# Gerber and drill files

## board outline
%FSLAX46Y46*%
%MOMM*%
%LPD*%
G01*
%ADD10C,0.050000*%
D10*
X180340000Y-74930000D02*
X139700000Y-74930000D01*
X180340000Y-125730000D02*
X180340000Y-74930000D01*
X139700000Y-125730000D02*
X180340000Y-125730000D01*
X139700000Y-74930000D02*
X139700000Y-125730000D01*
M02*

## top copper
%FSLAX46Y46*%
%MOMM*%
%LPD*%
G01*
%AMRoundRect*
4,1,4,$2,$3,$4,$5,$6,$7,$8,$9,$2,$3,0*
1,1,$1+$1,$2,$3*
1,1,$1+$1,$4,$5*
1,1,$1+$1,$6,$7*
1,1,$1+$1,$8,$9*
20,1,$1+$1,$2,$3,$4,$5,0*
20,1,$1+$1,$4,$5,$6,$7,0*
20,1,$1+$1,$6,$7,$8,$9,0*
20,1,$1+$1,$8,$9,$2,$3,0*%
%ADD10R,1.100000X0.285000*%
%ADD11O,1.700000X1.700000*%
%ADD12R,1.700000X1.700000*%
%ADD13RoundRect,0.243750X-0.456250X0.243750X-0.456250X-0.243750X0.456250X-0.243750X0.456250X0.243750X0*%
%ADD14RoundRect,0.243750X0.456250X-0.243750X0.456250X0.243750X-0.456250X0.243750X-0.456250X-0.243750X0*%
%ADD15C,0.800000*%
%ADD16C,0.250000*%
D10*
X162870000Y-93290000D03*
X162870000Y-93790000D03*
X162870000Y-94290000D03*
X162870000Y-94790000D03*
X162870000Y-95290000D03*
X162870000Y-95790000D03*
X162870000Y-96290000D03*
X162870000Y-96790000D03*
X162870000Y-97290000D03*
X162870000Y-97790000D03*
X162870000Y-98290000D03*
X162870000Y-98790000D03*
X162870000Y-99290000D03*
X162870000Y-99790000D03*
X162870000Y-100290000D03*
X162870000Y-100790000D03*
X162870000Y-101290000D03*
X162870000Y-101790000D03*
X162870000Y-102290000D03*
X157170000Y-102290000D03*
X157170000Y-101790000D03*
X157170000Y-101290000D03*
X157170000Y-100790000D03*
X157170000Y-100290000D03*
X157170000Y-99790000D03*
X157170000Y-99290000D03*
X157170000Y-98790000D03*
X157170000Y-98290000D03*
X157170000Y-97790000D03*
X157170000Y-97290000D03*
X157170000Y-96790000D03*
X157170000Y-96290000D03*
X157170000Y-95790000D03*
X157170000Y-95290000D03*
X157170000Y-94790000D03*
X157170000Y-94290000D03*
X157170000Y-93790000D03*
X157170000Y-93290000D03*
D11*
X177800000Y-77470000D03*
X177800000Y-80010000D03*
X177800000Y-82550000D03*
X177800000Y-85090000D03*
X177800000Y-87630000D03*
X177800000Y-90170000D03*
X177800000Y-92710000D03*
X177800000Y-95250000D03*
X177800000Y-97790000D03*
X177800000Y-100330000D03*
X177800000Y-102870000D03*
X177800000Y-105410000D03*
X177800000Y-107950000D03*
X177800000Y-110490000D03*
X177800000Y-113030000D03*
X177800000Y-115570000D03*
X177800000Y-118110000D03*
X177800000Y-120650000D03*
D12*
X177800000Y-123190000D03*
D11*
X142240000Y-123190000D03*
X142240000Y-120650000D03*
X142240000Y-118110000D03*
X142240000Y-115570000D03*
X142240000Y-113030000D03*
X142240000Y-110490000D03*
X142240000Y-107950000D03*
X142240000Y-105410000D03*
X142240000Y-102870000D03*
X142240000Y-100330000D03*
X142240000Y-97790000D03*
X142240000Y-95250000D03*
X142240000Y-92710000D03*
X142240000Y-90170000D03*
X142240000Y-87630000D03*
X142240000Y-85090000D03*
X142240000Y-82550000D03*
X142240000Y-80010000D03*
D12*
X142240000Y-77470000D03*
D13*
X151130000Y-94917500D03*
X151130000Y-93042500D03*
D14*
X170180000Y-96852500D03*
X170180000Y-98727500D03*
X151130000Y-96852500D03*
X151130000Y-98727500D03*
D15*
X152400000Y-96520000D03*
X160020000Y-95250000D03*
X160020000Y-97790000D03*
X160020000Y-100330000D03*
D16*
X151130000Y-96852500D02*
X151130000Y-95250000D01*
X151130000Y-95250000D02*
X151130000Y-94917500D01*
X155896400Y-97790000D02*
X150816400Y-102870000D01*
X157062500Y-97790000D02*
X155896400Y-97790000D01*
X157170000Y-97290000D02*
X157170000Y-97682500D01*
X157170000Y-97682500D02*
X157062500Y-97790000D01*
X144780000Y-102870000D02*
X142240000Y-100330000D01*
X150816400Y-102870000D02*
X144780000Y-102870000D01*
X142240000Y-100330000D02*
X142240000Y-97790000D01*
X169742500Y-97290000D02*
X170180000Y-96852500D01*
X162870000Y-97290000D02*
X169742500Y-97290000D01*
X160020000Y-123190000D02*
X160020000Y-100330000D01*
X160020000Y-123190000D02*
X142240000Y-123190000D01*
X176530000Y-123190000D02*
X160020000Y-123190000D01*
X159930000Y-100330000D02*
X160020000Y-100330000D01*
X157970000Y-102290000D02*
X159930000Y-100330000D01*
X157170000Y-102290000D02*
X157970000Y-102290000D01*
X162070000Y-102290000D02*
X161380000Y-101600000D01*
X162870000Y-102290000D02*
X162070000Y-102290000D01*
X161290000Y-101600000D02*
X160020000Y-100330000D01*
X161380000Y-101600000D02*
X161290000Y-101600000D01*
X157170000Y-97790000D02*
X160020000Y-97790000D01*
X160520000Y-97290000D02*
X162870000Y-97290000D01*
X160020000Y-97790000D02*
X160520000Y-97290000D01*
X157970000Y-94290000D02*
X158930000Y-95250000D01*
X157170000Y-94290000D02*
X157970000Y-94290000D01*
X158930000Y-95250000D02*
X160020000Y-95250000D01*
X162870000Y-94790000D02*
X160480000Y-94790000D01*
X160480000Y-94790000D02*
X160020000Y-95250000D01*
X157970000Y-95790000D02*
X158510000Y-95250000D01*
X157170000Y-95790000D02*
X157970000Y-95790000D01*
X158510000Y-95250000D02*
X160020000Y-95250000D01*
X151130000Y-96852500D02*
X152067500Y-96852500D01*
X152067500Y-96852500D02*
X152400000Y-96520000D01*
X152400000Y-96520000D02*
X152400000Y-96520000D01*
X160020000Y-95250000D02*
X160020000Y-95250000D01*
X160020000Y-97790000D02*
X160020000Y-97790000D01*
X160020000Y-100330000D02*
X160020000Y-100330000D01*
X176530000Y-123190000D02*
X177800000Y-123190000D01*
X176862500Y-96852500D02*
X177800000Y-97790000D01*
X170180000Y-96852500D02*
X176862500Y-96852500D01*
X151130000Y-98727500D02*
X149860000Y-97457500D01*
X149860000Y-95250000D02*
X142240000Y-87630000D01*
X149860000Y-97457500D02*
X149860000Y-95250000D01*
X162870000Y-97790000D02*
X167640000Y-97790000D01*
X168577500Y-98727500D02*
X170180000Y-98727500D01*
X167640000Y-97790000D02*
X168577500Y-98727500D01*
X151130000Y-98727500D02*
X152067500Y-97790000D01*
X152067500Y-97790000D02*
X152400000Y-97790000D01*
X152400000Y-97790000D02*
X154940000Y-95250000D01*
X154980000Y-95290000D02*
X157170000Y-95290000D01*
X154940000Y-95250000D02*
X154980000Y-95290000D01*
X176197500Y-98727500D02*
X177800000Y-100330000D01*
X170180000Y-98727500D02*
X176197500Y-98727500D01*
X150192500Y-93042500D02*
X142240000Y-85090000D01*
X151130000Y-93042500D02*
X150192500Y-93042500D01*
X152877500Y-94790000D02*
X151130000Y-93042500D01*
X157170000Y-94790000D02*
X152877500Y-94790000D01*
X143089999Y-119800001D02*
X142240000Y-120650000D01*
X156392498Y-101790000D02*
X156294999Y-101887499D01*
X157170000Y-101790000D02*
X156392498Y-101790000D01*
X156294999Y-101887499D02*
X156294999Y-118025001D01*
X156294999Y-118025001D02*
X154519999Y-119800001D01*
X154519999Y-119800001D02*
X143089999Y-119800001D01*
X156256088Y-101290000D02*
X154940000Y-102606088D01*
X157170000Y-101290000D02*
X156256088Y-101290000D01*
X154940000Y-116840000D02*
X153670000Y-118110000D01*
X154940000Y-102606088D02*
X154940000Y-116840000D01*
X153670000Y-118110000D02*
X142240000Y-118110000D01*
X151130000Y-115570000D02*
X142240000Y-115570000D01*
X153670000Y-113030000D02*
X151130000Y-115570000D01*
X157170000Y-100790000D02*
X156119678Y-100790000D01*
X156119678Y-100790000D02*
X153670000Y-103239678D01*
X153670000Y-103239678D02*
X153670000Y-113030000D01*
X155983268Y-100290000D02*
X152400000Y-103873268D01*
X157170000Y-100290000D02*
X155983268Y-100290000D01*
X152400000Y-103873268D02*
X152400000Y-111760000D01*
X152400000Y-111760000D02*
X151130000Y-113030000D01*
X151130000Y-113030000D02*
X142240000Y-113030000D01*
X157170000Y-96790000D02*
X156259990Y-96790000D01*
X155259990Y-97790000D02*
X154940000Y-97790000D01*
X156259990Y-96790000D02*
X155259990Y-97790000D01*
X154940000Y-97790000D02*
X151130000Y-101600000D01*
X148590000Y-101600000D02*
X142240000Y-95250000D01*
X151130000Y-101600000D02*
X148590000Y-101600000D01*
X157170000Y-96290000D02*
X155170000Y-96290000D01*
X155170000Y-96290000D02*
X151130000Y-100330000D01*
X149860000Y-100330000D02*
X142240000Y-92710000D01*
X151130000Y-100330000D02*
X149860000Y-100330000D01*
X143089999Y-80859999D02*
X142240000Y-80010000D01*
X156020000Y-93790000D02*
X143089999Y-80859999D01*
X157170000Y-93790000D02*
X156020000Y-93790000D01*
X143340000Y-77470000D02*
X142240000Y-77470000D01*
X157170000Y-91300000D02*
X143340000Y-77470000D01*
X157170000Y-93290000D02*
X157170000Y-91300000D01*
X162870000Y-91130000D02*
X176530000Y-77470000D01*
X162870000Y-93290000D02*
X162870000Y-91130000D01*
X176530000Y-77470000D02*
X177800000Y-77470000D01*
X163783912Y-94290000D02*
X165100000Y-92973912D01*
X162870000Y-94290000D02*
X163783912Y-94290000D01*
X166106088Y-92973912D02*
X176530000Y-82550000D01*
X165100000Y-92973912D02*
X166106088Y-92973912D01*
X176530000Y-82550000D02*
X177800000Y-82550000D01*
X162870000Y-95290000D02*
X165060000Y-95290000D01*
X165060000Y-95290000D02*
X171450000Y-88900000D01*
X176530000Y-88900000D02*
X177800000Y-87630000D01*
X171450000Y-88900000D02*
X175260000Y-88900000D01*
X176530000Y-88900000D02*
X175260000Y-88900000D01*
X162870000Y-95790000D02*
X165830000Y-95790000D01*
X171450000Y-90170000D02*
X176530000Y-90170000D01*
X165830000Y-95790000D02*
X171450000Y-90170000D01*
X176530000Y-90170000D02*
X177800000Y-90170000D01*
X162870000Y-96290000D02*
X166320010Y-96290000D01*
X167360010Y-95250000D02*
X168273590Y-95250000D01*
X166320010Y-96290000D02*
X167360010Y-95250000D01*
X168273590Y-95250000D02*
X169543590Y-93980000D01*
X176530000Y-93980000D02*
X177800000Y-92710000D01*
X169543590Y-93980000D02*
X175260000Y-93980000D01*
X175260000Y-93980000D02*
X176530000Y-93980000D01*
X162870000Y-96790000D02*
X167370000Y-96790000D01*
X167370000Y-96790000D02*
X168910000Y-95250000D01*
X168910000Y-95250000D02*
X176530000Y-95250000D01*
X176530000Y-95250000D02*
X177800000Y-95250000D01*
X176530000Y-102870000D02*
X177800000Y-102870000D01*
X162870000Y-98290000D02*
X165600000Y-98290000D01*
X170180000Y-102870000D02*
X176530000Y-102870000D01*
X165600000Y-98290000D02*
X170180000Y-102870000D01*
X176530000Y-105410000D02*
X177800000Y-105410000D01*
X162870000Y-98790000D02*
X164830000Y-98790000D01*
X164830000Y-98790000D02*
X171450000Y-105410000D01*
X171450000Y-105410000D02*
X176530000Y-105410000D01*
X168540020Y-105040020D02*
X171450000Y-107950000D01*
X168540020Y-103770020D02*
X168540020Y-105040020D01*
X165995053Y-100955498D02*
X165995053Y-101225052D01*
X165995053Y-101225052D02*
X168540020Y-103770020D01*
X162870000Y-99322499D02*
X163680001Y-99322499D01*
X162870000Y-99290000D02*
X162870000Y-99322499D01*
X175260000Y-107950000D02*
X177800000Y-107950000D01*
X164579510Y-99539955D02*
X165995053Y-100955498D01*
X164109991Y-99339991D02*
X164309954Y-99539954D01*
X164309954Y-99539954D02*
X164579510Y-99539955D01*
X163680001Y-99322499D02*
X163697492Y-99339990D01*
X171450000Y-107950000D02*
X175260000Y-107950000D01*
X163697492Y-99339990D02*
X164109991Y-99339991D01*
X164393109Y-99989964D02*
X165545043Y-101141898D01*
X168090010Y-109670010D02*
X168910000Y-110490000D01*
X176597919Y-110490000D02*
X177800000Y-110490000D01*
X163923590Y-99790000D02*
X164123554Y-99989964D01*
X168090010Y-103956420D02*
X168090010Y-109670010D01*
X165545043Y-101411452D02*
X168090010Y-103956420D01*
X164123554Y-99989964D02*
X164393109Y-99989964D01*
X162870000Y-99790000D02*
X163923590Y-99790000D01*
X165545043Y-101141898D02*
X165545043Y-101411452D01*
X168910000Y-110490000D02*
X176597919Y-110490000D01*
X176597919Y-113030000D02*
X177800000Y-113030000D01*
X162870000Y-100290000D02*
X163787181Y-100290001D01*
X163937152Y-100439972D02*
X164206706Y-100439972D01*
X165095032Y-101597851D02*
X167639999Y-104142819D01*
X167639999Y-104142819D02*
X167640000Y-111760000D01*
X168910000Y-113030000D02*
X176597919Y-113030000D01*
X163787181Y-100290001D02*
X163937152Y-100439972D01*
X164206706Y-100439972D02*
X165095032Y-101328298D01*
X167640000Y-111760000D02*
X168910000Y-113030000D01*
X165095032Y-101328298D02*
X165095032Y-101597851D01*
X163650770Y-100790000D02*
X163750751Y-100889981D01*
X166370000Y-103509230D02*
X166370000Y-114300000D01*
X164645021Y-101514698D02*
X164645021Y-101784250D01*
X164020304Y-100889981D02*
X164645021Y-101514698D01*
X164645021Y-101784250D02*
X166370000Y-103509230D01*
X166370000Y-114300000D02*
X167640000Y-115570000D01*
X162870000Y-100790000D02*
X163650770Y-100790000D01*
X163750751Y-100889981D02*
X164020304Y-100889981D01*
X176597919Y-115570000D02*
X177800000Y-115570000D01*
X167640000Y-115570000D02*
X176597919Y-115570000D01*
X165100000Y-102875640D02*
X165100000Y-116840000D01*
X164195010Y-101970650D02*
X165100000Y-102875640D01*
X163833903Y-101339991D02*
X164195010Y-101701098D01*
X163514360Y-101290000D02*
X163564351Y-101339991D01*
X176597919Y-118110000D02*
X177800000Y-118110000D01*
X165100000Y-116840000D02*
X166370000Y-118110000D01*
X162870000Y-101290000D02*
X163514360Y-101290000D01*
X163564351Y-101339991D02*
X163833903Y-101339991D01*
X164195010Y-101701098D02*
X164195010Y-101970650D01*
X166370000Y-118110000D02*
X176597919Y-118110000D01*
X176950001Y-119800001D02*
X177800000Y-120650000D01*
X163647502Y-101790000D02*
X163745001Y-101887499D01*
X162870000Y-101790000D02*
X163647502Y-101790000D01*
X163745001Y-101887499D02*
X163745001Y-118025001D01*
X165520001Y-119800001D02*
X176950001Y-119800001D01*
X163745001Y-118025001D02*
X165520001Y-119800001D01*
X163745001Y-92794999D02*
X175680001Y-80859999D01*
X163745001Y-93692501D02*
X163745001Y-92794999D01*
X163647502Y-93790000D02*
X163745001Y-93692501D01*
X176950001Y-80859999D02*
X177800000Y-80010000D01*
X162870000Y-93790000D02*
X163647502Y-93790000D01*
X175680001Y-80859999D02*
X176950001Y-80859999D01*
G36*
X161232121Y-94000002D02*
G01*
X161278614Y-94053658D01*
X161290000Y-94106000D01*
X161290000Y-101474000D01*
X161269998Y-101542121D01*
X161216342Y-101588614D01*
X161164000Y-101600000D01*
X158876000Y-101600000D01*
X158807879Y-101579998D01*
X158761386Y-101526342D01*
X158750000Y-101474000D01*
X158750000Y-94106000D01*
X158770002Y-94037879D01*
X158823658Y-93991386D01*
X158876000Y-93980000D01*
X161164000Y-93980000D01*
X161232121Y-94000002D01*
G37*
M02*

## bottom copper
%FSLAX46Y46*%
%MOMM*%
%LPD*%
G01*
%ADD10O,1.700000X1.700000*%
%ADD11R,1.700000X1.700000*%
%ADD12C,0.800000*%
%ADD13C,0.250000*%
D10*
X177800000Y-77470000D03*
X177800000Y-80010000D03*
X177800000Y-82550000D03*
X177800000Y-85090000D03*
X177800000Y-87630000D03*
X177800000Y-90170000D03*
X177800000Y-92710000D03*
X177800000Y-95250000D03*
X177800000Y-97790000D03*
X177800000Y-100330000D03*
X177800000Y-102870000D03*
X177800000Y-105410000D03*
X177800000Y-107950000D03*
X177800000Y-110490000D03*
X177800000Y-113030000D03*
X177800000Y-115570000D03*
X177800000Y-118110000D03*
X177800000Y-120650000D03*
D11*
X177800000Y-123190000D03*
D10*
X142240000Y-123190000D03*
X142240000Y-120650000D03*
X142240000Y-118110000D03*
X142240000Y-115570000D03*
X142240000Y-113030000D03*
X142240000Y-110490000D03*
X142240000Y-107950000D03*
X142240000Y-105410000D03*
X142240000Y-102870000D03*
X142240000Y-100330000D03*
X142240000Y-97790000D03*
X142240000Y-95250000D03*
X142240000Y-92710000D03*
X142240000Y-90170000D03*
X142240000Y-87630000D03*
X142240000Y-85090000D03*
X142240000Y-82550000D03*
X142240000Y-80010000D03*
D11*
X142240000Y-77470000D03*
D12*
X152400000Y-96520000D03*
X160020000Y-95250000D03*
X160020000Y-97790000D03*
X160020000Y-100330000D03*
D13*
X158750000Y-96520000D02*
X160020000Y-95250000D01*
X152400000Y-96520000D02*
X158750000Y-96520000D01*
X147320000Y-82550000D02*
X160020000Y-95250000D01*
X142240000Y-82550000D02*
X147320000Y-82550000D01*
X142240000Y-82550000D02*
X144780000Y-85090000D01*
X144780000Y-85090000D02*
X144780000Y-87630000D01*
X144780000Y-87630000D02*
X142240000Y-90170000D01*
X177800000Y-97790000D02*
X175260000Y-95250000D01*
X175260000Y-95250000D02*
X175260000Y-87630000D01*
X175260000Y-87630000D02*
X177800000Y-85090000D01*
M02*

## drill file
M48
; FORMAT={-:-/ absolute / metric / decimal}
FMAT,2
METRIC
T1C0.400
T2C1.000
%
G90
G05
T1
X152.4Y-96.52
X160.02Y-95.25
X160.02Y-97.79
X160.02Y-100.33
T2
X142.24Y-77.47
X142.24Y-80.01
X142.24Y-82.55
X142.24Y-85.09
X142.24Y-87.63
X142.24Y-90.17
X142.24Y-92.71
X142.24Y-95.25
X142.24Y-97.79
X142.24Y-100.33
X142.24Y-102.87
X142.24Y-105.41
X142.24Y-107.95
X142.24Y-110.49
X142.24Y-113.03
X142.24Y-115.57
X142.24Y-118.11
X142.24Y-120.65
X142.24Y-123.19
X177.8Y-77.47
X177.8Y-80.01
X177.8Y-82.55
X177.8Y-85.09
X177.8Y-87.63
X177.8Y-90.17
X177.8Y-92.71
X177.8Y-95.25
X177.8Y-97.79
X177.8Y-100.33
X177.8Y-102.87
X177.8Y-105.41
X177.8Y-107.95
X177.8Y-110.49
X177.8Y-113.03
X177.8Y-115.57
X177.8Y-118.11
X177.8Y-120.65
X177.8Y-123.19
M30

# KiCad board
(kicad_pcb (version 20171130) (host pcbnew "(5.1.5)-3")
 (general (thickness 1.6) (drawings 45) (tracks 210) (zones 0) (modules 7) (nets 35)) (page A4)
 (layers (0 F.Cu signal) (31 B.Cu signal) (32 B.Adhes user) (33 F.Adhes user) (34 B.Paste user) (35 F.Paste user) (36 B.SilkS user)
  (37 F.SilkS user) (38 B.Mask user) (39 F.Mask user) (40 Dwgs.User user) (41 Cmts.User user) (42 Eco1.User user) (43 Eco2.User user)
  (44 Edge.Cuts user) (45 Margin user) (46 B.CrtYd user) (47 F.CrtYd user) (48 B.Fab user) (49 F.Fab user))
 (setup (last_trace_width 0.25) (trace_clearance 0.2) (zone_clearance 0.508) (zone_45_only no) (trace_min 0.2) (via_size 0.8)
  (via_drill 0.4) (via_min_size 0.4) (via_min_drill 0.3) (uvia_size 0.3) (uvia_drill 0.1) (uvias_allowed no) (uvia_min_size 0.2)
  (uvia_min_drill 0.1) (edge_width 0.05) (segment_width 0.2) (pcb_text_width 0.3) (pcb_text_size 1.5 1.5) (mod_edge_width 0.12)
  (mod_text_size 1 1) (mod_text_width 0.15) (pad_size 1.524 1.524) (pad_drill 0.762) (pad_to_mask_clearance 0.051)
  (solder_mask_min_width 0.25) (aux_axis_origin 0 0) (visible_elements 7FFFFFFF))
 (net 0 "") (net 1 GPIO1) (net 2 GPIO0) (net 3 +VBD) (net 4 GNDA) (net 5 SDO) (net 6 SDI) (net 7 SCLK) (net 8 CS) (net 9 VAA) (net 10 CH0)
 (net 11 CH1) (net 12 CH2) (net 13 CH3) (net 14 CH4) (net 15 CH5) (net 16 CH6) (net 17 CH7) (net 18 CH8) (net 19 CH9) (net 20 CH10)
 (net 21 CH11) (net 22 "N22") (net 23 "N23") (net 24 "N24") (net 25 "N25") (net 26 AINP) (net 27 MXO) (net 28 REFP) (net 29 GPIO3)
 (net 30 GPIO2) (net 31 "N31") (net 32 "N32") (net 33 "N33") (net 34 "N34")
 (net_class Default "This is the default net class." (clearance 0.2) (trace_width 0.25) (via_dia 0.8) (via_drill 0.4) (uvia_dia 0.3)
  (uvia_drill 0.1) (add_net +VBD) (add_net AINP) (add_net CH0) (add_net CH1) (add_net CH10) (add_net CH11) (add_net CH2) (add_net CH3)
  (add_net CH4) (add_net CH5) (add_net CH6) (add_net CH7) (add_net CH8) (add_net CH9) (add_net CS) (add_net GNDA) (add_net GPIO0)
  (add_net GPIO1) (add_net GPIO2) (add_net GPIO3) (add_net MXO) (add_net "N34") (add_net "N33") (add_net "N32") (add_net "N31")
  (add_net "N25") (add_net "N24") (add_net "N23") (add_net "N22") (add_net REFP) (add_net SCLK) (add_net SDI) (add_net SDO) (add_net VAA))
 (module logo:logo (layer F.Cu) (at 160.02 82.55)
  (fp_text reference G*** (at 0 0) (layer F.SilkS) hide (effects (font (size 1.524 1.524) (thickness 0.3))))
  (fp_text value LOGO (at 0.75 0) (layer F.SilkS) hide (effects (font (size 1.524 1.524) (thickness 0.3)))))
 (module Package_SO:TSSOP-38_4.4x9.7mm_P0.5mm (layer F.Cu) (at 160.02 97.79)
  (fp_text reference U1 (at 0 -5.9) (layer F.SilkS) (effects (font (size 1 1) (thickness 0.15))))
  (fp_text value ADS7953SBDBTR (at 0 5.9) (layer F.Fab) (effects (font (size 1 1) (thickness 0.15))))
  (pad 38 smd rect (at 2.85 -4.5) (size 1.1 0.285) (layers F.Cu F.Paste F.Mask) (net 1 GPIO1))
  (pad 37 smd rect (at 2.85 -4) (size 1.1 0.285) (layers F.Cu F.Paste F.Mask) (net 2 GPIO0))
  (pad 36 smd rect (at 2.85 -3.5) (size 1.1 0.285) (layers F.Cu F.Paste F.Mask) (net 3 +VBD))
  (pad 35 smd rect (at 2.85 -3) (size 1.1 0.285) (layers F.Cu F.Paste F.Mask) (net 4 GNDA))
  (pad 34 smd rect (at 2.85 -2.5) (size 1.1 0.285) (layers F.Cu F.Paste F.Mask) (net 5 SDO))
  (pad 33 smd rect (at 2.85 -2) (size 1.1 0.285) (layers F.Cu F.Paste F.Mask) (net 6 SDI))
  (pad 32 smd rect (at 2.85 -1.5) (size 1.1 0.285) (layers F.Cu F.Paste F.Mask) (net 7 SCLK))
  (pad 31 smd rect (at 2.85 -1) (size 1.1 0.285) (layers F.Cu F.Paste F.Mask) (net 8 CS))
  (pad 30 smd rect (at 2.85 -0.5) (size 1.1 0.285) (layers F.Cu F.Paste F.Mask) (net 4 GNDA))
  (pad 29 smd rect (at 2.85 0) (size 1.1 0.285) (layers F.Cu F.Paste F.Mask) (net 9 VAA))
  (pad 28 smd rect (at 2.85 0.5) (size 1.1 0.285) (layers F.Cu F.Paste F.Mask) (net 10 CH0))
  (pad 27 smd rect (at 2.85 1) (size 1.1 0.285) (layers F.Cu F.Paste F.Mask) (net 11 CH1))
  (pad 26 smd rect (at 2.85 1.5) (size 1.1 0.285) (layers F.Cu F.Paste F.Mask) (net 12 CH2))
  (pad 25 smd rect (at 2.85 2) (size 1.1 0.285) (layers F.Cu F.Paste F.Mask) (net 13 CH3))
  (pad 24 smd rect (at 2.85 2.5) (size 1.1 0.285) (layers F.Cu F.Paste F.Mask) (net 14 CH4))
  (pad 23 smd rect (at 2.85 3) (size 1.1 0.285) (layers F.Cu F.Paste F.Mask) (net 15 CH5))
  (pad 22 smd rect (at 2.85 3.5) (size 1.1 0.285) (layers F.Cu F.Paste F.Mask) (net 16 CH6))
  (pad 21 smd rect (at 2.85 4) (size 1.1 0.285) (layers F.Cu F.Paste F.Mask) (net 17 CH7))
  (pad 20 smd rect (at 2.85 4.5) (size 1.1 0.285) (layers F.Cu F.Paste F.Mask) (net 4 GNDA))
  (pad 19 smd rect (at -2.85 4.5) (size 1.1 0.285) (layers F.Cu F.Paste F.Mask) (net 4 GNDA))
  (pad 18 smd rect (at -2.85 4) (size 1.1 0.285) (layers F.Cu F.Paste F.Mask) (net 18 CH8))
  (pad 17 smd rect (at -2.85 3.5) (size 1.1 0.285) (layers F.Cu F.Paste F.Mask) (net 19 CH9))
  (pad 16 smd rect (at -2.85 3) (size 1.1 0.285) (layers F.Cu F.Paste F.Mask) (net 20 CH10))
  (pad 15 smd rect (at -2.85 2.5) (size 1.1 0.285) (layers F.Cu F.Paste F.Mask) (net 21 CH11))
  (pad 14 smd rect (at -2.85 2) (size 1.1 0.285) (layers F.Cu F.Paste F.Mask) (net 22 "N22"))
  (pad 13 smd rect (at -2.85 1.5) (size 1.1 0.285) (layers F.Cu F.Paste F.Mask) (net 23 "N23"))
  (pad 12 smd rect (at -2.85 1) (size 1.1 0.285) (layers F.Cu F.Paste F.Mask) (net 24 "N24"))
  (pad 11 smd rect (at -2.85 0.5) (size 1.1 0.285) (layers F.Cu F.Paste F.Mask) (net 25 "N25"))
  (pad 10 smd rect (at -2.85 0) (size 1.1 0.285) (layers F.Cu F.Paste F.Mask) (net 4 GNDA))
  (pad 9 smd rect (at -2.85 -0.5) (size 1.1 0.285) (layers F.Cu F.Paste F.Mask) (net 4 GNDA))
  (pad 8 smd rect (at -2.85 -1) (size 1.1 0.285) (layers F.Cu F.Paste F.Mask) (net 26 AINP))
  (pad 7 smd rect (at -2.85 -1.5) (size 1.1 0.285) (layers F.Cu F.Paste F.Mask) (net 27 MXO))
  (pad 6 smd rect (at -2.85 -2) (size 1.1 0.285) (layers F.Cu F.Paste F.Mask) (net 4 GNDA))
  (pad 5 smd rect (at -2.85 -2.5) (size 1.1 0.285) (layers F.Cu F.Paste F.Mask) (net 9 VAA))
  (pad 4 smd rect (at -2.85 -3) (size 1.1 0.285) (layers F.Cu F.Paste F.Mask) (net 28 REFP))
  (pad 3 smd rect (at -2.85 -3.5) (size 1.1 0.285) (layers F.Cu F.Paste F.Mask) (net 4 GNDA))
  (pad 2 smd rect (at -2.85 -4) (size 1.1 0.285) (layers F.Cu F.Paste F.Mask) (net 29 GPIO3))
  (pad 1 smd rect (at -2.85 -4.5) (size 1.1 0.285) (layers F.Cu F.Paste F.Mask) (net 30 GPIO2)))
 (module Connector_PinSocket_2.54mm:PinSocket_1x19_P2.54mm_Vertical (layer F.Cu) (at 177.8 123.19 180)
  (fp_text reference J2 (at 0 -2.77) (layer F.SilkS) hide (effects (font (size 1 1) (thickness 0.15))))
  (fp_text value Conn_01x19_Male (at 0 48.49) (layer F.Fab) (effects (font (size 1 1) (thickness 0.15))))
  (pad 19 thru_hole oval (at 0 45.72 180) (size 1.7 1.7) (drill 1) (layers *.Cu *.Mask) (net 1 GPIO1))
  (pad 18 thru_hole oval (at 0 43.18 180) (size 1.7 1.7) (drill 1) (layers *.Cu *.Mask) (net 2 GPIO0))
  (pad 17 thru_hole oval (at 0 40.64 180) (size 1.7 1.7) (drill 1) (layers *.Cu *.Mask) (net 3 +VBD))
  (pad 16 thru_hole oval (at 0 38.1 180) (size 1.7 1.7) (drill 1) (layers *.Cu *.Mask) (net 4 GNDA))
  (pad 15 thru_hole oval (at 0 35.56 180) (size 1.7 1.7) (drill 1) (layers *.Cu *.Mask) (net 5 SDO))
  (pad 14 thru_hole oval (at 0 33.02 180) (size 1.7 1.7) (drill 1) (layers *.Cu *.Mask) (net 6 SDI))
  (pad 13 thru_hole oval (at 0 30.48 180) (size 1.7 1.7) (drill 1) (layers *.Cu *.Mask) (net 7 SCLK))
  (pad 12 thru_hole oval (at 0 27.94 180) (size 1.7 1.7) (drill 1) (layers *.Cu *.Mask) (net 8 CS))
  (pad 11 thru_hole oval (at 0 25.4 180) (size 1.7 1.7) (drill 1) (layers *.Cu *.Mask) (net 4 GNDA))
  (pad 10 thru_hole oval (at 0 22.86 180) (size 1.7 1.7) (drill 1) (layers *.Cu *.Mask) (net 9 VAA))
  (pad 9 thru_hole oval (at 0 20.32 180) (size 1.7 1.7) (drill 1) (layers *.Cu *.Mask) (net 10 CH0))
  (pad 8 thru_hole oval (at 0 17.78 180) (size 1.7 1.7) (drill 1) (layers *.Cu *.Mask) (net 11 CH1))
  (pad 7 thru_hole oval (at 0 15.24 180) (size 1.7 1.7) (drill 1) (layers *.Cu *.Mask) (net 12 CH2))
  (pad 6 thru_hole oval (at 0 12.7 180) (size 1.7 1.7) (drill 1) (layers *.Cu *.Mask) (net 13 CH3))
  (pad 5 thru_hole oval (at 0 10.16 180) (size 1.7 1.7) (drill 1) (layers *.Cu *.Mask) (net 14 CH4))
  (pad 4 thru_hole oval (at 0 7.62 180) (size 1.7 1.7) (drill 1) (layers *.Cu *.Mask) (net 15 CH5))
  (pad 3 thru_hole oval (at 0 5.08 180) (size 1.7 1.7) (drill 1) (layers *.Cu *.Mask) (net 16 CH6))
  (pad 2 thru_hole oval (at 0 2.54 180) (size 1.7 1.7) (drill 1) (layers *.Cu *.Mask) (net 17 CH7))
  (pad 1 thru_hole rect (at 0 0 180) (size 1.7 1.7) (drill 1) (layers *.Cu *.Mask) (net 4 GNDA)))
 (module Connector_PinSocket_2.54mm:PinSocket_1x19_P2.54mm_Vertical (layer F.Cu) (at 142.24 77.47)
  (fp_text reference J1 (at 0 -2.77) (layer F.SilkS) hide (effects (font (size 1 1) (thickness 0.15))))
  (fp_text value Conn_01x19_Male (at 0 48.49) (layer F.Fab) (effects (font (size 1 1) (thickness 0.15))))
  (pad 19 thru_hole oval (at 0 45.72) (size 1.7 1.7) (drill 1) (layers *.Cu *.Mask) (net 4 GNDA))
  (pad 18 thru_hole oval (at 0 43.18) (size 1.7 1.7) (drill 1) (layers *.Cu *.Mask) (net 18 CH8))
  (pad 17 thru_hole oval (at 0 40.64) (size 1.7 1.7) (drill 1) (layers *.Cu *.Mask) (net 19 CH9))
  (pad 16 thru_hole oval (at 0 38.1) (size 1.7 1.7) (drill 1) (layers *.Cu *.Mask) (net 20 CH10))
  (pad 15 thru_hole oval (at 0 35.56) (size 1.7 1.7) (drill 1) (layers *.Cu *.Mask) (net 21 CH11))
  (pad 14 thru_hole oval (at 0 33.02) (size 1.7 1.7) (drill 1) (layers *.Cu *.Mask) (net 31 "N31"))
  (pad 13 thru_hole oval (at 0 30.48) (size 1.7 1.7) (drill 1) (layers *.Cu *.Mask) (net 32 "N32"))
  (pad 12 thru_hole oval (at 0 27.94) (size 1.7 1.7) (drill 1) (layers *.Cu *.Mask) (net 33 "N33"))
  (pad 11 thru_hole oval (at 0 25.4) (size 1.7 1.7) (drill 1) (layers *.Cu *.Mask) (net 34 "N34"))
  (pad 10 thru_hole oval (at 0 22.86) (size 1.7 1.7) (drill 1) (layers *.Cu *.Mask) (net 4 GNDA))
  (pad 9 thru_hole oval (at 0 20.32) (size 1.7 1.7) (drill 1) (layers *.Cu *.Mask) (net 4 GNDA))
  (pad 8 thru_hole oval (at 0 17.78) (size 1.7 1.7) (drill 1) (layers *.Cu *.Mask) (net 26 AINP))
  (pad 7 thru_hole oval (at 0 15.24) (size 1.7 1.7) (drill 1) (layers *.Cu *.Mask) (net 27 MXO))
  (pad 6 thru_hole oval (at 0 12.7) (size 1.7 1.7) (drill 1) (layers *.Cu *.Mask) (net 4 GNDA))
  (pad 5 thru_hole oval (at 0 10.16) (size 1.7 1.7) (drill 1) (layers *.Cu *.Mask) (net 9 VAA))
  (pad 4 thru_hole oval (at 0 7.62) (size 1.7 1.7) (drill 1) (layers *.Cu *.Mask) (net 28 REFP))
  (pad 3 thru_hole oval (at 0 5.08) (size 1.7 1.7) (drill 1) (layers *.Cu *.Mask) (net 4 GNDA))
  (pad 2 thru_hole oval (at 0 2.54) (size 1.7 1.7) (drill 1) (layers *.Cu *.Mask) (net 29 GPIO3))
  (pad 1 thru_hole rect (at 0 0) (size 1.7 1.7) (drill 1) (layers *.Cu *.Mask) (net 30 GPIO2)))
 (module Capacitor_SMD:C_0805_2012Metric (layer F.Cu) (at 151.13 93.98 270)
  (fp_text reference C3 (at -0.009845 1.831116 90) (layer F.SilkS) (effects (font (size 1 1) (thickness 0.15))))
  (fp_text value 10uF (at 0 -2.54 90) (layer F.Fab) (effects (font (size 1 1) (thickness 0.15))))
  (pad 2 smd roundrect (at 0.9375 0 270) (size 0.975 1.4) (layers F.Cu F.Paste F.Mask) (roundrect_rratio 0.25) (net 4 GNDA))
  (pad 1 smd roundrect (at -0.9375 0 270) (size 0.975 1.4) (layers F.Cu F.Paste F.Mask) (roundrect_rratio 0.25) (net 28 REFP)))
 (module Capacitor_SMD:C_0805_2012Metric (layer F.Cu) (at 170.18 97.79 90)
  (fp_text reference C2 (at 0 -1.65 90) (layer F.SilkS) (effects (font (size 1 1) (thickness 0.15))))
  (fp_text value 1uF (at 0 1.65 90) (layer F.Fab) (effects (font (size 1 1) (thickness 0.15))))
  (pad 2 smd roundrect (at 0.9375 0 90) (size 0.975 1.4) (layers F.Cu F.Paste F.Mask) (roundrect_rratio 0.25) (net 4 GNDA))
  (pad 1 smd roundrect (at -0.9375 0 90) (size 0.975 1.4) (layers F.Cu F.Paste F.Mask) (roundrect_rratio 0.25) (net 9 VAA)))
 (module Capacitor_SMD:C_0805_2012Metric (layer F.Cu) (at 151.13 97.79 90)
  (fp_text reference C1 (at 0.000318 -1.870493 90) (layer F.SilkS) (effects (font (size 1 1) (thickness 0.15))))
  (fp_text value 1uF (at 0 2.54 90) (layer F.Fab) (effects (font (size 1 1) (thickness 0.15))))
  (pad 2 smd roundrect (at 0.9375 0 90) (size 0.975 1.4) (layers F.Cu F.Paste F.Mask) (roundrect_rratio 0.25) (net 4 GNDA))
  (pad 1 smd roundrect (at -0.9375 0 90) (size 0.975 1.4) (layers F.Cu F.Paste F.Mask) (roundrect_rratio 0.25) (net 9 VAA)))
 (gr_line (start 180.34 74.93) (end 139.7 74.93) (layer Edge.Cuts) (width 0.05))
 (gr_line (start 180.34 125.73) (end 180.34 74.93) (layer Edge.Cuts) (width 0.05))
 (gr_line (start 139.7 125.73) (end 180.34 125.73) (layer Edge.Cuts) (width 0.05))
 (gr_line (start 139.7 74.93) (end 139.7 125.73) (layer Edge.Cuts) (width 0.05))
 (segment (start 151.13 96.8525) (end 151.13 95.25) (width 0.25) (layer F.Cu) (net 4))
 (segment (start 151.13 95.25) (end 151.13 94.9175) (width 0.25) (layer F.Cu) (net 4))
 (segment (start 155.8964 97.79) (end 150.8164 102.87) (width 0.25) (layer F.Cu) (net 4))
 (segment (start 157.0625 97.79) (end 155.8964 97.79) (width 0.25) (layer F.Cu) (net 4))
 (segment (start 157.17 97.29) (end 157.17 97.6825) (width 0.25) (layer F.Cu) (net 4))
 (segment (start 157.17 97.6825) (end 157.0625 97.79) (width 0.25) (layer F.Cu) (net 4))
 (segment (start 144.78 102.87) (end 142.24 100.33) (width 0.25) (layer F.Cu) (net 4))
 (segment (start 150.8164 102.87) (end 144.78 102.87) (width 0.25) (layer F.Cu) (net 4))
 (segment (start 142.24 100.33) (end 142.24 97.79) (width 0.25) (layer F.Cu) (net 4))
 (segment (start 169.7425 97.29) (end 170.18 96.8525) (width 0.25) (layer F.Cu) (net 4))
 (segment (start 162.87 97.29) (end 169.7425 97.29) (width 0.25) (layer F.Cu) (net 4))
 (segment (start 160.02 123.19) (end 160.02 100.33) (width 0.25) (layer F.Cu) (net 4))
 (segment (start 160.02 123.19) (end 142.24 123.19) (width 0.25) (layer F.Cu) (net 4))
 (segment (start 176.53 123.19) (end 160.02 123.19) (width 0.25) (layer F.Cu) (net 4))
 (segment (start 159.93 100.33) (end 160.02 100.33) (width 0.25) (layer F.Cu) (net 4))
 (segment (start 157.97 102.29) (end 159.93 100.33) (width 0.25) (layer F.Cu) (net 4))
 (segment (start 157.17 102.29) (end 157.97 102.29) (width 0.25) (layer F.Cu) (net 4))
 (segment (start 162.07 102.29) (end 161.38 101.6) (width 0.25) (layer F.Cu) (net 4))
 (segment (start 162.87 102.29) (end 162.07 102.29) (width 0.25) (layer F.Cu) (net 4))
 (segment (start 161.29 101.6) (end 160.02 100.33) (width 0.25) (layer F.Cu) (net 4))
 (segment (start 161.38 101.6) (end 161.29 101.6) (width 0.25) (layer F.Cu) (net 4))
 (segment (start 157.17 97.79) (end 160.02 97.79) (width 0.25) (layer F.Cu) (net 4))
 (segment (start 160.52 97.29) (end 162.87 97.29) (width 0.25) (layer F.Cu) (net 4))
 (segment (start 160.02 97.79) (end 160.52 97.29) (width 0.25) (layer F.Cu) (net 4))
 (segment (start 157.97 94.29) (end 158.93 95.25) (width 0.25) (layer F.Cu) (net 4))
 (segment (start 157.17 94.29) (end 157.97 94.29) (width 0.25) (layer F.Cu) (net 4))
 (segment (start 158.93 95.25) (end 160.02 95.25) (width 0.25) (layer F.Cu) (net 4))
 (segment (start 162.87 94.79) (end 160.48 94.79) (width 0.25) (layer F.Cu) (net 4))
 (segment (start 160.48 94.79) (end 160.02 95.25) (width 0.25) (layer F.Cu) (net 4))
 (segment (start 157.97 95.79) (end 158.51 95.25) (width 0.25) (layer F.Cu) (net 4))
 (segment (start 157.17 95.79) (end 157.97 95.79) (width 0.25) (layer F.Cu) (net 4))
 (segment (start 158.51 95.25) (end 160.02 95.25) (width 0.25) (layer F.Cu) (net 4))
 (segment (start 151.13 96.8525) (end 152.0675 96.8525) (width 0.25) (layer F.Cu) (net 4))
 (segment (start 152.0675 96.8525) (end 152.4 96.52) (width 0.25) (layer F.Cu) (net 4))
 (segment (start 152.4 96.52) (end 152.4 96.52) (width 0.25) (layer F.Cu) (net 4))
 (via (at 152.4 96.52) (size 0.8) (drill 0.4) (layers F.Cu B.Cu) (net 4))
 (segment (start 160.02 95.25) (end 160.02 95.25) (width 0.25) (layer F.Cu) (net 4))
 (via (at 160.02 95.25) (size 0.8) (drill 0.4) (layers F.Cu B.Cu) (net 4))
 (segment (start 160.02 97.79) (end 160.02 97.79) (width 0.25) (layer F.Cu) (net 4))
 (via (at 160.02 97.79) (size 0.8) (drill 0.4) (layers F.Cu B.Cu) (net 4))
 (segment (start 160.02 100.33) (end 160.02 100.33) (width 0.25) (layer F.Cu) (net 4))
 (via (at 160.02 100.33) (size 0.8) (drill 0.4) (layers F.Cu B.Cu) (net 4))
 (segment (start 158.75 96.52) (end 160.02 95.25) (width 0.25) (layer B.Cu) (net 4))
 (segment (start 152.4 96.52) (end 158.75 96.52) (width 0.25) (layer B.Cu) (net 4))
 (segment (start 147.32 82.55) (end 160.02 95.25) (width 0.25) (layer B.Cu) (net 4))
 (segment (start 142.24 82.55) (end 147.32 82.55) (width 0.25) (layer B.Cu) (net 4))
 (segment (start 176.53 123.19) (end 177.8 123.19) (width 0.25) (layer F.Cu) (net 4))
 (segment (start 176.8625 96.8525) (end 177.8 97.79) (width 0.25) (layer F.Cu) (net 4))
 (segment (start 170.18 96.8525) (end 176.8625 96.8525) (width 0.25) (layer F.Cu) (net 4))
 (segment (start 142.24 82.55) (end 144.78 85.09) (width 0.25) (layer B.Cu) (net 4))
 (segment (start 144.78 85.09) (end 144.78 87.63) (width 0.25) (layer B.Cu) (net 4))
 (segment (start 144.78 87.63) (end 142.24 90.17) (width 0.25) (layer B.Cu) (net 4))
 (segment (start 177.8 97.79) (end 175.26 95.25) (width 0.25) (layer B.Cu) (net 4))
 (segment (start 175.26 95.25) (end 175.26 87.63) (width 0.25) (layer B.Cu) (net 4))
 (segment (start 175.26 87.63) (end 177.8 85.09) (width 0.25) (layer B.Cu) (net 4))
 (segment (start 151.13 98.7275) (end 149.86 97.4575) (width 0.25) (layer F.Cu) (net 9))
 (segment (start 149.86 95.25) (end 142.24 87.63) (width 0.25) (layer F.Cu) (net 9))
 (segment (start 149.86 97.4575) (end 149.86 95.25) (width 0.25) (layer F.Cu) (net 9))
 (segment (start 162.87 97.79) (end 167.64 97.79) (width 0.25) (layer F.Cu) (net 9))
 (segment (start 168.5775 98.7275) (end 170.18 98.7275) (width 0.25) (layer F.Cu) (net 9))
 (segment (start 167.64 97.79) (end 168.5775 98.7275) (width 0.25) (layer F.Cu) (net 9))
 (segment (start 151.13 98.7275) (end 152.0675 97.79) (width 0.25) (layer F.Cu) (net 9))
 (segment (start 152.0675 97.79) (end 152.4 97.79) (width 0.25) (layer F.Cu) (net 9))
 (segment (start 152.4 97.79) (end 154.94 95.25) (width 0.25) (layer F.Cu) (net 9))
 (segment (start 154.98 95.29) (end 157.17 95.29) (width 0.25) (layer F.Cu) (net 9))
 (segment (start 154.94 95.25) (end 154.98 95.29) (width 0.25) (layer F.Cu) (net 9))
 (segment (start 176.1975 98.7275) (end 177.8 100.33) (width 0.25) (layer F.Cu) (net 9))
 (segment (start 170.18 98.7275) (end 176.1975 98.7275) (width 0.25) (layer F.Cu) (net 9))
 (segment (start 150.1925 93.0425) (end 142.24 85.09) (width 0.25) (layer F.Cu) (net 28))
 (segment (start 151.13 93.0425) (end 150.1925 93.0425) (width 0.25) (layer F.Cu) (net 28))
 (segment (start 152.8775 94.79) (end 151.13 93.0425) (width 0.25) (layer F.Cu) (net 28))
 (segment (start 157.17 94.79) (end 152.8775 94.79) (width 0.25) (layer F.Cu) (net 28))
 (segment (start 143.089999 119.800001) (end 142.24 120.65) (width 0.25) (layer F.Cu) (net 18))
 (segment (start 156.392498 101.79) (end 156.294999 101.887499) (width 0.25) (layer F.Cu) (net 18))
 (segment (start 157.17 101.79) (end 156.392498 101.79) (width 0.25) (layer F.Cu) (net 18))
 (segment (start 156.294999 101.887499) (end 156.294999 118.025001) (width 0.25) (layer F.Cu) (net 18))
 (segment (start 156.294999 118.025001) (end 154.519999 119.800001) (width 0.25) (layer F.Cu) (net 18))
 (segment (start 154.519999 119.800001) (end 143.089999 119.800001) (width 0.25) (layer F.Cu) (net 18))
 (segment (start 156.256088 101.29) (end 154.94 102.606088) (width 0.25) (layer F.Cu) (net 19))
 (segment (start 157.17 101.29) (end 156.256088 101.29) (width 0.25) (layer F.Cu) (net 19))
 (segment (start 154.94 116.84) (end 153.67 118.11) (width 0.25) (layer F.Cu) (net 19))
 (segment (start 154.94 102.606088) (end 154.94 116.84) (width 0.25) (layer F.Cu) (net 19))
 (segment (start 153.67 118.11) (end 142.24 118.11) (width 0.25) (layer F.Cu) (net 19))
 (segment (start 151.13 115.57) (end 142.24 115.57) (width 0.25) (layer F.Cu) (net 20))
 (segment (start 153.67 113.03) (end 151.13 115.57) (width 0.25) (layer F.Cu) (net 20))
 (segment (start 157.17 100.79) (end 156.119678 100.79) (width 0.25) (layer F.Cu) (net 20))
 (segment (start 156.119678 100.79) (end 153.67 103.239678) (width 0.25) (layer F.Cu) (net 20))
 (segment (start 153.67 103.239678) (end 153.67 113.03) (width 0.25) (layer F.Cu) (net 20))
 (segment (start 155.983268 100.29) (end 152.4 103.873268) (width 0.25) (layer F.Cu) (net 21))
 (segment (start 157.17 100.29) (end 155.983268 100.29) (width 0.25) (layer F.Cu) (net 21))
 (segment (start 152.4 103.873268) (end 152.4 111.76) (width 0.25) (layer F.Cu) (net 21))
 (segment (start 152.4 111.76) (end 151.13 113.03) (width 0.25) (layer F.Cu) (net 21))
 (segment (start 151.13 113.03) (end 142.24 113.03) (width 0.25) (layer F.Cu) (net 21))
 (segment (start 157.17 96.79) (end 156.25999 96.79) (width 0.25) (layer F.Cu) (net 26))
 (segment (start 155.25999 97.79) (end 154.94 97.79) (width 0.25) (layer F.Cu) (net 26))
 (segment (start 156.25999 96.79) (end 155.25999 97.79) (width 0.25) (layer F.Cu) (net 26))
 (segment (start 154.94 97.79) (end 151.13 101.6) (width 0.25) (layer F.Cu) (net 26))
 (segment (start 148.59 101.6) (end 142.24 95.25) (width 0.25) (layer F.Cu) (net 26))
 (segment (start 151.13 101.6) (end 148.59 101.6) (width 0.25) (layer F.Cu) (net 26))
 (segment (start 157.17 96.29) (end 155.17 96.29) (width 0.25) (layer F.Cu) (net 27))
 (segment (start 155.17 96.29) (end 151.13 100.33) (width 0.25) (layer F.Cu) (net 27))
 (segment (start 149.86 100.33) (end 142.24 92.71) (width 0.25) (layer F.Cu) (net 27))
 (segment (start 151.13 100.33) (end 149.86 100.33) (width 0.25) (layer F.Cu) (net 27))
 (segment (start 143.089999 80.859999) (end 142.24 80.01) (width 0.25) (layer F.Cu) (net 29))
 (segment (start 156.02 93.79) (end 143.089999 80.859999) (width 0.25) (layer F.Cu) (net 29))
 (segment (start 157.17 93.79) (end 156.02 93.79) (width 0.25) (layer F.Cu) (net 29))
 (segment (start 143.34 77.47) (end 142.24 77.47) (width 0.25) (layer F.Cu) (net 30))
 (segment (start 157.17 91.3) (end 143.34 77.47) (width 0.25) (layer F.Cu) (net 30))
 (segment (start 157.17 93.29) (end 157.17 91.3) (width 0.25) (layer F.Cu) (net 30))
 (segment (start 162.87 91.13) (end 176.53 77.47) (width 0.25) (layer F.Cu) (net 1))
 (segment (start 162.87 93.29) (end 162.87 91.13) (width 0.25) (layer F.Cu) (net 1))
 (segment (start 176.53 77.47) (end 177.8 77.47) (width 0.25) (layer F.Cu) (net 1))
 (segment (start 163.783912 94.29) (end 165.1 92.973912) (width 0.25) (layer F.Cu) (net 3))
 (segment (start 162.87 94.29) (end 163.783912 94.29) (width 0.25) (layer F.Cu) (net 3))
 (segment (start 166.106088 92.973912) (end 176.53 82.55) (width 0.25) (layer F.Cu) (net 3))
 (segment (start 165.1 92.973912) (end 166.106088 92.973912) (width 0.25) (layer F.Cu) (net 3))
 (segment (start 176.53 82.55) (end 177.8 82.55) (width 0.25) (layer F.Cu) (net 3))
 (segment (start 162.87 95.29) (end 165.06 95.29) (width 0.25) (layer F.Cu) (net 5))
 (segment (start 165.06 95.29) (end 171.45 88.9) (width 0.25) (layer F.Cu) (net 5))
 (segment (start 176.53 88.9) (end 177.8 87.63) (width 0.25) (layer F.Cu) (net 5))
 (segment (start 171.45 88.9) (end 175.26 88.9) (width 0.25) (layer F.Cu) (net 5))
 (segment (start 176.53 88.9) (end 175.26 88.9) (width 0.25) (layer F.Cu) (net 5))
 (segment (start 162.87 95.79) (end 165.83 95.79) (width 0.25) (layer F.Cu) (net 6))
 (segment (start 171.45 90.17) (end 176.53 90.17) (width 0.25) (layer F.Cu) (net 6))
 (segment (start 165.83 95.79) (end 171.45 90.17) (width 0.25) (layer F.Cu) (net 6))
 (segment (start 176.53 90.17) (end 177.8 90.17) (width 0.25) (layer F.Cu) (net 6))
 (segment (start 162.87 96.29) (end 166.32001 96.29) (width 0.25) (layer F.Cu) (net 7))
 (segment (start 167.36001 95.25) (end 168.27359 95.25) (width 0.25) (layer F.Cu) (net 7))
 (segment (start 166.32001 96.29) (end 167.36001 95.25) (width 0.25) (layer F.Cu) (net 7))
 (segment (start 168.27359 95.25) (end 169.54359 93.98) (width 0.25) (layer F.Cu) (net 7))
 (segment (start 176.53 93.98) (end 177.8 92.71) (width 0.25) (layer F.Cu) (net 7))
 (segment (start 169.54359 93.98) (end 175.26 93.98) (width 0.25) (layer F.Cu) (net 7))
 (segment (start 175.26 93.98) (end 176.53 93.98) (width 0.25) (layer F.Cu) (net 7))
 (segment (start 162.87 96.79) (end 167.37 96.79) (width 0.25) (layer F.Cu) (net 8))
 (segment (start 167.37 96.79) (end 168.91 95.25) (width 0.25) (layer F.Cu) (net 8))
 (segment (start 168.91 95.25) (end 176.53 95.25) (width 0.25) (layer F.Cu) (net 8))
 (segment (start 176.53 95.25) (end 177.8 95.25) (width 0.25) (layer F.Cu) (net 8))
 (segment (start 176.53 102.87) (end 177.8 102.87) (width 0.25) (layer F.Cu) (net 10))
 (segment (start 162.87 98.29) (end 165.6 98.29) (width 0.25) (layer F.Cu) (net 10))
 (segment (start 170.18 102.87) (end 176.53 102.87) (width 0.25) (layer F.Cu) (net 10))
 (segment (start 165.6 98.29) (end 170.18 102.87) (width 0.25) (layer F.Cu) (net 10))
 (segment (start 176.53 105.41) (end 177.8 105.41) (width 0.25) (layer F.Cu) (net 11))
 (segment (start 162.87 98.79) (end 164.83 98.79) (width 0.25) (layer F.Cu) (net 11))
 (segment (start 164.83 98.79) (end 171.45 105.41) (width 0.25) (layer F.Cu) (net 11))
 (segment (start 171.45 105.41) (end 176.53 105.41) (width 0.25) (layer F.Cu) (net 11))
 (segment (start 168.54002 105.04002) (end 171.45 107.95) (width 0.25) (layer F.Cu) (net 12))
 (segment (start 168.54002 103.77002) (end 168.54002 105.04002) (width 0.25) (layer F.Cu) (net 12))
 (segment (start 165.995053 100.955498) (end 165.995053 101.225052) (width 0.25) (layer F.Cu) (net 12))
 (segment (start 165.995053 101.225052) (end 168.54002 103.77002) (width 0.25) (layer F.Cu) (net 12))
 (segment (start 162.87 99.322499) (end 163.680001 99.322499) (width 0.25) (layer F.Cu) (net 12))
 (segment (start 162.87 99.29) (end 162.87 99.322499) (width 0.25) (layer F.Cu) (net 12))
 (segment (start 175.26 107.95) (end 177.8 107.95) (width 0.25) (layer F.Cu) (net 12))
 (segment (start 164.57951 99.539955) (end 165.995053 100.955498) (width 0.25) (layer F.Cu) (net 12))
 (segment (start 164.109991 99.339991) (end 164.309954 99.539954) (width 0.25) (layer F.Cu) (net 12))
 (segment (start 164.309954 99.539954) (end 164.57951 99.539955) (width 0.25) (layer F.Cu) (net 12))
 (segment (start 163.680001 99.322499) (end 163.697492 99.33999) (width 0.25) (layer F.Cu) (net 12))
 (segment (start 171.45 107.95) (end 175.26 107.95) (width 0.25) (layer F.Cu) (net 12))
 (segment (start 163.697492 99.33999) (end 164.109991 99.339991) (width 0.25) (layer F.Cu) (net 12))
 (segment (start 164.393109 99.989964) (end 165.545043 101.141898) (width 0.25) (layer F.Cu) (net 13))
 (segment (start 168.09001 109.67001) (end 168.91 110.49) (width 0.25) (layer F.Cu) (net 13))
 (segment (start 176.597919 110.49) (end 177.8 110.49) (width 0.25) (layer F.Cu) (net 13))
 (segment (start 163.92359 99.79) (end 164.123554 99.989964) (width 0.25) (layer F.Cu) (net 13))
 (segment (start 168.09001 103.95642) (end 168.09001 109.67001) (width 0.25) (layer F.Cu) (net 13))
 (segment (start 165.545043 101.411452) (end 168.09001 103.95642) (width 0.25) (layer F.Cu) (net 13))
 (segment (start 164.123554 99.989964) (end 164.393109 99.989964) (width 0.25) (layer F.Cu) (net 13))
 (segment (start 162.87 99.79) (end 163.92359 99.79) (width 0.25) (layer F.Cu) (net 13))
 (segment (start 165.545043 101.141898) (end 165.545043 101.411452) (width 0.25) (layer F.Cu) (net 13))
 (segment (start 168.91 110.49) (end 176.597919 110.49) (width 0.25) (layer F.Cu) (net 13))
 (segment (start 176.597919 113.03) (end 177.8 113.03) (width 0.25) (layer F.Cu) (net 14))
 (segment (start 162.87 100.29) (end 163.787181 100.290001) (width 0.25) (layer F.Cu) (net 14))
 (segment (start 163.937152 100.439972) (end 164.206706 100.439972) (width 0.25) (layer F.Cu) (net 14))
 (segment (start 165.095032 101.597851) (end 167.639999 104.142819) (width 0.25) (layer F.Cu) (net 14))
 (segment (start 167.639999 104.142819) (end 167.64 111.76) (width 0.25) (layer F.Cu) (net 14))
 (segment (start 168.91 113.03) (end 176.597919 113.03) (width 0.25) (layer F.Cu) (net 14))
 (segment (start 163.787181 100.290001) (end 163.937152 100.439972) (width 0.25) (layer F.Cu) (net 14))
 (segment (start 164.206706 100.439972) (end 165.095032 101.328298) (width 0.25) (layer F.Cu) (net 14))
 (segment (start 167.64 111.76) (end 168.91 113.03) (width 0.25) (layer F.Cu) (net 14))
 (segment (start 165.095032 101.328298) (end 165.095032 101.597851) (width 0.25) (layer F.Cu) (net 14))
 (segment (start 163.65077 100.79) (end 163.750751 100.889981) (width 0.25) (layer F.Cu) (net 15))
 (segment (start 166.37 103.50923) (end 166.37 114.3) (width 0.25) (layer F.Cu) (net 15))
 (segment (start 164.645021 101.514698) (end 164.645021 101.78425) (width 0.25) (layer F.Cu) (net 15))
 (segment (start 164.020304 100.889981) (end 164.645021 101.514698) (width 0.25) (layer F.Cu) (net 15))
 (segment (start 164.645021 101.78425) (end 166.37 103.50923) (width 0.25) (layer F.Cu) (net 15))
 (segment (start 166.37 114.3) (end 167.64 115.57) (width 0.25) (layer F.Cu) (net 15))
 (segment (start 162.87 100.79) (end 163.65077 100.79) (width 0.25) (layer F.Cu) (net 15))
 (segment (start 163.750751 100.889981) (end 164.020304 100.889981) (width 0.25) (layer F.Cu) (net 15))
 (segment (start 176.597919 115.57) (end 177.8 115.57) (width 0.25) (layer F.Cu) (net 15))
 (segment (start 167.64 115.57) (end 176.597919 115.57) (width 0.25) (layer F.Cu) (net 15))
 (segment (start 165.1 102.87564) (end 165.1 116.84) (width 0.25) (layer F.Cu) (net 16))
 (segment (start 164.19501 101.97065) (end 165.1 102.87564) (width 0.25) (layer F.Cu) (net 16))
 (segment (start 163.833903 101.339991) (end 164.19501 101.701098) (width 0.25) (layer F.Cu) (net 16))
 (segment (start 163.51436 101.29) (end 163.564351 101.339991) (width 0.25) (layer F.Cu) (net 16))
 (segment (start 176.597919 118.11) (end 177.8 118.11) (width 0.25) (layer F.Cu) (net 16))
 (segment (start 165.1 116.84) (end 166.37 118.11) (width 0.25) (layer F.Cu) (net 16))
 (segment (start 162.87 101.29) (end 163.51436 101.29) (width 0.25) (layer F.Cu) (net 16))
 (segment (start 163.564351 101.339991) (end 163.833903 101.339991) (width 0.25) (layer F.Cu) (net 16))
 (segment (start 164.19501 101.701098) (end 164.19501 101.97065) (width 0.25) (layer F.Cu) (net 16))
 (segment (start 166.37 118.11) (end 176.597919 118.11) (width 0.25) (layer F.Cu) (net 16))
 (segment (start 176.950001 119.800001) (end 177.8 120.65) (width 0.25) (layer F.Cu) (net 17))
 (segment (start 163.647502 101.79) (end 163.745001 101.887499) (width 0.25) (layer F.Cu) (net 17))
 (segment (start 162.87 101.79) (end 163.647502 101.79) (width 0.25) (layer F.Cu) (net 17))
 (segment (start 163.745001 101.887499) (end 163.745001 118.025001) (width 0.25) (layer F.Cu) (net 17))
 (segment (start 165.520001 119.800001) (end 176.950001 119.800001) (width 0.25) (layer F.Cu) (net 17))
 (segment (start 163.745001 118.025001) (end 165.520001 119.800001) (width 0.25) (layer F.Cu) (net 17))
 (segment (start 163.745001 92.794999) (end 175.680001 80.859999) (width 0.25) (layer F.Cu) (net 2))
 (segment (start 163.745001 93.692501) (end 163.745001 92.794999) (width 0.25) (layer F.Cu) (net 2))
 (segment (start 163.647502 93.79) (end 163.745001 93.692501) (width 0.25) (layer F.Cu) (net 2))
 (segment (start 176.950001 80.859999) (end 177.8 80.01) (width 0.25) (layer F.Cu) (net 2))
 (segment (start 162.87 93.79) (end 163.647502 93.79) (width 0.25) (layer F.Cu) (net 2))
 (segment (start 175.680001 80.859999) (end 176.950001 80.859999) (width 0.25) (layer F.Cu) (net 2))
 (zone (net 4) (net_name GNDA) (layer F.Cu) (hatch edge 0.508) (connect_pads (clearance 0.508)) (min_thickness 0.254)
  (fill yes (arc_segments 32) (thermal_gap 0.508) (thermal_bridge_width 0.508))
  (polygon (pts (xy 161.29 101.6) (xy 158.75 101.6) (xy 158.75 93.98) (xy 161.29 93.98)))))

